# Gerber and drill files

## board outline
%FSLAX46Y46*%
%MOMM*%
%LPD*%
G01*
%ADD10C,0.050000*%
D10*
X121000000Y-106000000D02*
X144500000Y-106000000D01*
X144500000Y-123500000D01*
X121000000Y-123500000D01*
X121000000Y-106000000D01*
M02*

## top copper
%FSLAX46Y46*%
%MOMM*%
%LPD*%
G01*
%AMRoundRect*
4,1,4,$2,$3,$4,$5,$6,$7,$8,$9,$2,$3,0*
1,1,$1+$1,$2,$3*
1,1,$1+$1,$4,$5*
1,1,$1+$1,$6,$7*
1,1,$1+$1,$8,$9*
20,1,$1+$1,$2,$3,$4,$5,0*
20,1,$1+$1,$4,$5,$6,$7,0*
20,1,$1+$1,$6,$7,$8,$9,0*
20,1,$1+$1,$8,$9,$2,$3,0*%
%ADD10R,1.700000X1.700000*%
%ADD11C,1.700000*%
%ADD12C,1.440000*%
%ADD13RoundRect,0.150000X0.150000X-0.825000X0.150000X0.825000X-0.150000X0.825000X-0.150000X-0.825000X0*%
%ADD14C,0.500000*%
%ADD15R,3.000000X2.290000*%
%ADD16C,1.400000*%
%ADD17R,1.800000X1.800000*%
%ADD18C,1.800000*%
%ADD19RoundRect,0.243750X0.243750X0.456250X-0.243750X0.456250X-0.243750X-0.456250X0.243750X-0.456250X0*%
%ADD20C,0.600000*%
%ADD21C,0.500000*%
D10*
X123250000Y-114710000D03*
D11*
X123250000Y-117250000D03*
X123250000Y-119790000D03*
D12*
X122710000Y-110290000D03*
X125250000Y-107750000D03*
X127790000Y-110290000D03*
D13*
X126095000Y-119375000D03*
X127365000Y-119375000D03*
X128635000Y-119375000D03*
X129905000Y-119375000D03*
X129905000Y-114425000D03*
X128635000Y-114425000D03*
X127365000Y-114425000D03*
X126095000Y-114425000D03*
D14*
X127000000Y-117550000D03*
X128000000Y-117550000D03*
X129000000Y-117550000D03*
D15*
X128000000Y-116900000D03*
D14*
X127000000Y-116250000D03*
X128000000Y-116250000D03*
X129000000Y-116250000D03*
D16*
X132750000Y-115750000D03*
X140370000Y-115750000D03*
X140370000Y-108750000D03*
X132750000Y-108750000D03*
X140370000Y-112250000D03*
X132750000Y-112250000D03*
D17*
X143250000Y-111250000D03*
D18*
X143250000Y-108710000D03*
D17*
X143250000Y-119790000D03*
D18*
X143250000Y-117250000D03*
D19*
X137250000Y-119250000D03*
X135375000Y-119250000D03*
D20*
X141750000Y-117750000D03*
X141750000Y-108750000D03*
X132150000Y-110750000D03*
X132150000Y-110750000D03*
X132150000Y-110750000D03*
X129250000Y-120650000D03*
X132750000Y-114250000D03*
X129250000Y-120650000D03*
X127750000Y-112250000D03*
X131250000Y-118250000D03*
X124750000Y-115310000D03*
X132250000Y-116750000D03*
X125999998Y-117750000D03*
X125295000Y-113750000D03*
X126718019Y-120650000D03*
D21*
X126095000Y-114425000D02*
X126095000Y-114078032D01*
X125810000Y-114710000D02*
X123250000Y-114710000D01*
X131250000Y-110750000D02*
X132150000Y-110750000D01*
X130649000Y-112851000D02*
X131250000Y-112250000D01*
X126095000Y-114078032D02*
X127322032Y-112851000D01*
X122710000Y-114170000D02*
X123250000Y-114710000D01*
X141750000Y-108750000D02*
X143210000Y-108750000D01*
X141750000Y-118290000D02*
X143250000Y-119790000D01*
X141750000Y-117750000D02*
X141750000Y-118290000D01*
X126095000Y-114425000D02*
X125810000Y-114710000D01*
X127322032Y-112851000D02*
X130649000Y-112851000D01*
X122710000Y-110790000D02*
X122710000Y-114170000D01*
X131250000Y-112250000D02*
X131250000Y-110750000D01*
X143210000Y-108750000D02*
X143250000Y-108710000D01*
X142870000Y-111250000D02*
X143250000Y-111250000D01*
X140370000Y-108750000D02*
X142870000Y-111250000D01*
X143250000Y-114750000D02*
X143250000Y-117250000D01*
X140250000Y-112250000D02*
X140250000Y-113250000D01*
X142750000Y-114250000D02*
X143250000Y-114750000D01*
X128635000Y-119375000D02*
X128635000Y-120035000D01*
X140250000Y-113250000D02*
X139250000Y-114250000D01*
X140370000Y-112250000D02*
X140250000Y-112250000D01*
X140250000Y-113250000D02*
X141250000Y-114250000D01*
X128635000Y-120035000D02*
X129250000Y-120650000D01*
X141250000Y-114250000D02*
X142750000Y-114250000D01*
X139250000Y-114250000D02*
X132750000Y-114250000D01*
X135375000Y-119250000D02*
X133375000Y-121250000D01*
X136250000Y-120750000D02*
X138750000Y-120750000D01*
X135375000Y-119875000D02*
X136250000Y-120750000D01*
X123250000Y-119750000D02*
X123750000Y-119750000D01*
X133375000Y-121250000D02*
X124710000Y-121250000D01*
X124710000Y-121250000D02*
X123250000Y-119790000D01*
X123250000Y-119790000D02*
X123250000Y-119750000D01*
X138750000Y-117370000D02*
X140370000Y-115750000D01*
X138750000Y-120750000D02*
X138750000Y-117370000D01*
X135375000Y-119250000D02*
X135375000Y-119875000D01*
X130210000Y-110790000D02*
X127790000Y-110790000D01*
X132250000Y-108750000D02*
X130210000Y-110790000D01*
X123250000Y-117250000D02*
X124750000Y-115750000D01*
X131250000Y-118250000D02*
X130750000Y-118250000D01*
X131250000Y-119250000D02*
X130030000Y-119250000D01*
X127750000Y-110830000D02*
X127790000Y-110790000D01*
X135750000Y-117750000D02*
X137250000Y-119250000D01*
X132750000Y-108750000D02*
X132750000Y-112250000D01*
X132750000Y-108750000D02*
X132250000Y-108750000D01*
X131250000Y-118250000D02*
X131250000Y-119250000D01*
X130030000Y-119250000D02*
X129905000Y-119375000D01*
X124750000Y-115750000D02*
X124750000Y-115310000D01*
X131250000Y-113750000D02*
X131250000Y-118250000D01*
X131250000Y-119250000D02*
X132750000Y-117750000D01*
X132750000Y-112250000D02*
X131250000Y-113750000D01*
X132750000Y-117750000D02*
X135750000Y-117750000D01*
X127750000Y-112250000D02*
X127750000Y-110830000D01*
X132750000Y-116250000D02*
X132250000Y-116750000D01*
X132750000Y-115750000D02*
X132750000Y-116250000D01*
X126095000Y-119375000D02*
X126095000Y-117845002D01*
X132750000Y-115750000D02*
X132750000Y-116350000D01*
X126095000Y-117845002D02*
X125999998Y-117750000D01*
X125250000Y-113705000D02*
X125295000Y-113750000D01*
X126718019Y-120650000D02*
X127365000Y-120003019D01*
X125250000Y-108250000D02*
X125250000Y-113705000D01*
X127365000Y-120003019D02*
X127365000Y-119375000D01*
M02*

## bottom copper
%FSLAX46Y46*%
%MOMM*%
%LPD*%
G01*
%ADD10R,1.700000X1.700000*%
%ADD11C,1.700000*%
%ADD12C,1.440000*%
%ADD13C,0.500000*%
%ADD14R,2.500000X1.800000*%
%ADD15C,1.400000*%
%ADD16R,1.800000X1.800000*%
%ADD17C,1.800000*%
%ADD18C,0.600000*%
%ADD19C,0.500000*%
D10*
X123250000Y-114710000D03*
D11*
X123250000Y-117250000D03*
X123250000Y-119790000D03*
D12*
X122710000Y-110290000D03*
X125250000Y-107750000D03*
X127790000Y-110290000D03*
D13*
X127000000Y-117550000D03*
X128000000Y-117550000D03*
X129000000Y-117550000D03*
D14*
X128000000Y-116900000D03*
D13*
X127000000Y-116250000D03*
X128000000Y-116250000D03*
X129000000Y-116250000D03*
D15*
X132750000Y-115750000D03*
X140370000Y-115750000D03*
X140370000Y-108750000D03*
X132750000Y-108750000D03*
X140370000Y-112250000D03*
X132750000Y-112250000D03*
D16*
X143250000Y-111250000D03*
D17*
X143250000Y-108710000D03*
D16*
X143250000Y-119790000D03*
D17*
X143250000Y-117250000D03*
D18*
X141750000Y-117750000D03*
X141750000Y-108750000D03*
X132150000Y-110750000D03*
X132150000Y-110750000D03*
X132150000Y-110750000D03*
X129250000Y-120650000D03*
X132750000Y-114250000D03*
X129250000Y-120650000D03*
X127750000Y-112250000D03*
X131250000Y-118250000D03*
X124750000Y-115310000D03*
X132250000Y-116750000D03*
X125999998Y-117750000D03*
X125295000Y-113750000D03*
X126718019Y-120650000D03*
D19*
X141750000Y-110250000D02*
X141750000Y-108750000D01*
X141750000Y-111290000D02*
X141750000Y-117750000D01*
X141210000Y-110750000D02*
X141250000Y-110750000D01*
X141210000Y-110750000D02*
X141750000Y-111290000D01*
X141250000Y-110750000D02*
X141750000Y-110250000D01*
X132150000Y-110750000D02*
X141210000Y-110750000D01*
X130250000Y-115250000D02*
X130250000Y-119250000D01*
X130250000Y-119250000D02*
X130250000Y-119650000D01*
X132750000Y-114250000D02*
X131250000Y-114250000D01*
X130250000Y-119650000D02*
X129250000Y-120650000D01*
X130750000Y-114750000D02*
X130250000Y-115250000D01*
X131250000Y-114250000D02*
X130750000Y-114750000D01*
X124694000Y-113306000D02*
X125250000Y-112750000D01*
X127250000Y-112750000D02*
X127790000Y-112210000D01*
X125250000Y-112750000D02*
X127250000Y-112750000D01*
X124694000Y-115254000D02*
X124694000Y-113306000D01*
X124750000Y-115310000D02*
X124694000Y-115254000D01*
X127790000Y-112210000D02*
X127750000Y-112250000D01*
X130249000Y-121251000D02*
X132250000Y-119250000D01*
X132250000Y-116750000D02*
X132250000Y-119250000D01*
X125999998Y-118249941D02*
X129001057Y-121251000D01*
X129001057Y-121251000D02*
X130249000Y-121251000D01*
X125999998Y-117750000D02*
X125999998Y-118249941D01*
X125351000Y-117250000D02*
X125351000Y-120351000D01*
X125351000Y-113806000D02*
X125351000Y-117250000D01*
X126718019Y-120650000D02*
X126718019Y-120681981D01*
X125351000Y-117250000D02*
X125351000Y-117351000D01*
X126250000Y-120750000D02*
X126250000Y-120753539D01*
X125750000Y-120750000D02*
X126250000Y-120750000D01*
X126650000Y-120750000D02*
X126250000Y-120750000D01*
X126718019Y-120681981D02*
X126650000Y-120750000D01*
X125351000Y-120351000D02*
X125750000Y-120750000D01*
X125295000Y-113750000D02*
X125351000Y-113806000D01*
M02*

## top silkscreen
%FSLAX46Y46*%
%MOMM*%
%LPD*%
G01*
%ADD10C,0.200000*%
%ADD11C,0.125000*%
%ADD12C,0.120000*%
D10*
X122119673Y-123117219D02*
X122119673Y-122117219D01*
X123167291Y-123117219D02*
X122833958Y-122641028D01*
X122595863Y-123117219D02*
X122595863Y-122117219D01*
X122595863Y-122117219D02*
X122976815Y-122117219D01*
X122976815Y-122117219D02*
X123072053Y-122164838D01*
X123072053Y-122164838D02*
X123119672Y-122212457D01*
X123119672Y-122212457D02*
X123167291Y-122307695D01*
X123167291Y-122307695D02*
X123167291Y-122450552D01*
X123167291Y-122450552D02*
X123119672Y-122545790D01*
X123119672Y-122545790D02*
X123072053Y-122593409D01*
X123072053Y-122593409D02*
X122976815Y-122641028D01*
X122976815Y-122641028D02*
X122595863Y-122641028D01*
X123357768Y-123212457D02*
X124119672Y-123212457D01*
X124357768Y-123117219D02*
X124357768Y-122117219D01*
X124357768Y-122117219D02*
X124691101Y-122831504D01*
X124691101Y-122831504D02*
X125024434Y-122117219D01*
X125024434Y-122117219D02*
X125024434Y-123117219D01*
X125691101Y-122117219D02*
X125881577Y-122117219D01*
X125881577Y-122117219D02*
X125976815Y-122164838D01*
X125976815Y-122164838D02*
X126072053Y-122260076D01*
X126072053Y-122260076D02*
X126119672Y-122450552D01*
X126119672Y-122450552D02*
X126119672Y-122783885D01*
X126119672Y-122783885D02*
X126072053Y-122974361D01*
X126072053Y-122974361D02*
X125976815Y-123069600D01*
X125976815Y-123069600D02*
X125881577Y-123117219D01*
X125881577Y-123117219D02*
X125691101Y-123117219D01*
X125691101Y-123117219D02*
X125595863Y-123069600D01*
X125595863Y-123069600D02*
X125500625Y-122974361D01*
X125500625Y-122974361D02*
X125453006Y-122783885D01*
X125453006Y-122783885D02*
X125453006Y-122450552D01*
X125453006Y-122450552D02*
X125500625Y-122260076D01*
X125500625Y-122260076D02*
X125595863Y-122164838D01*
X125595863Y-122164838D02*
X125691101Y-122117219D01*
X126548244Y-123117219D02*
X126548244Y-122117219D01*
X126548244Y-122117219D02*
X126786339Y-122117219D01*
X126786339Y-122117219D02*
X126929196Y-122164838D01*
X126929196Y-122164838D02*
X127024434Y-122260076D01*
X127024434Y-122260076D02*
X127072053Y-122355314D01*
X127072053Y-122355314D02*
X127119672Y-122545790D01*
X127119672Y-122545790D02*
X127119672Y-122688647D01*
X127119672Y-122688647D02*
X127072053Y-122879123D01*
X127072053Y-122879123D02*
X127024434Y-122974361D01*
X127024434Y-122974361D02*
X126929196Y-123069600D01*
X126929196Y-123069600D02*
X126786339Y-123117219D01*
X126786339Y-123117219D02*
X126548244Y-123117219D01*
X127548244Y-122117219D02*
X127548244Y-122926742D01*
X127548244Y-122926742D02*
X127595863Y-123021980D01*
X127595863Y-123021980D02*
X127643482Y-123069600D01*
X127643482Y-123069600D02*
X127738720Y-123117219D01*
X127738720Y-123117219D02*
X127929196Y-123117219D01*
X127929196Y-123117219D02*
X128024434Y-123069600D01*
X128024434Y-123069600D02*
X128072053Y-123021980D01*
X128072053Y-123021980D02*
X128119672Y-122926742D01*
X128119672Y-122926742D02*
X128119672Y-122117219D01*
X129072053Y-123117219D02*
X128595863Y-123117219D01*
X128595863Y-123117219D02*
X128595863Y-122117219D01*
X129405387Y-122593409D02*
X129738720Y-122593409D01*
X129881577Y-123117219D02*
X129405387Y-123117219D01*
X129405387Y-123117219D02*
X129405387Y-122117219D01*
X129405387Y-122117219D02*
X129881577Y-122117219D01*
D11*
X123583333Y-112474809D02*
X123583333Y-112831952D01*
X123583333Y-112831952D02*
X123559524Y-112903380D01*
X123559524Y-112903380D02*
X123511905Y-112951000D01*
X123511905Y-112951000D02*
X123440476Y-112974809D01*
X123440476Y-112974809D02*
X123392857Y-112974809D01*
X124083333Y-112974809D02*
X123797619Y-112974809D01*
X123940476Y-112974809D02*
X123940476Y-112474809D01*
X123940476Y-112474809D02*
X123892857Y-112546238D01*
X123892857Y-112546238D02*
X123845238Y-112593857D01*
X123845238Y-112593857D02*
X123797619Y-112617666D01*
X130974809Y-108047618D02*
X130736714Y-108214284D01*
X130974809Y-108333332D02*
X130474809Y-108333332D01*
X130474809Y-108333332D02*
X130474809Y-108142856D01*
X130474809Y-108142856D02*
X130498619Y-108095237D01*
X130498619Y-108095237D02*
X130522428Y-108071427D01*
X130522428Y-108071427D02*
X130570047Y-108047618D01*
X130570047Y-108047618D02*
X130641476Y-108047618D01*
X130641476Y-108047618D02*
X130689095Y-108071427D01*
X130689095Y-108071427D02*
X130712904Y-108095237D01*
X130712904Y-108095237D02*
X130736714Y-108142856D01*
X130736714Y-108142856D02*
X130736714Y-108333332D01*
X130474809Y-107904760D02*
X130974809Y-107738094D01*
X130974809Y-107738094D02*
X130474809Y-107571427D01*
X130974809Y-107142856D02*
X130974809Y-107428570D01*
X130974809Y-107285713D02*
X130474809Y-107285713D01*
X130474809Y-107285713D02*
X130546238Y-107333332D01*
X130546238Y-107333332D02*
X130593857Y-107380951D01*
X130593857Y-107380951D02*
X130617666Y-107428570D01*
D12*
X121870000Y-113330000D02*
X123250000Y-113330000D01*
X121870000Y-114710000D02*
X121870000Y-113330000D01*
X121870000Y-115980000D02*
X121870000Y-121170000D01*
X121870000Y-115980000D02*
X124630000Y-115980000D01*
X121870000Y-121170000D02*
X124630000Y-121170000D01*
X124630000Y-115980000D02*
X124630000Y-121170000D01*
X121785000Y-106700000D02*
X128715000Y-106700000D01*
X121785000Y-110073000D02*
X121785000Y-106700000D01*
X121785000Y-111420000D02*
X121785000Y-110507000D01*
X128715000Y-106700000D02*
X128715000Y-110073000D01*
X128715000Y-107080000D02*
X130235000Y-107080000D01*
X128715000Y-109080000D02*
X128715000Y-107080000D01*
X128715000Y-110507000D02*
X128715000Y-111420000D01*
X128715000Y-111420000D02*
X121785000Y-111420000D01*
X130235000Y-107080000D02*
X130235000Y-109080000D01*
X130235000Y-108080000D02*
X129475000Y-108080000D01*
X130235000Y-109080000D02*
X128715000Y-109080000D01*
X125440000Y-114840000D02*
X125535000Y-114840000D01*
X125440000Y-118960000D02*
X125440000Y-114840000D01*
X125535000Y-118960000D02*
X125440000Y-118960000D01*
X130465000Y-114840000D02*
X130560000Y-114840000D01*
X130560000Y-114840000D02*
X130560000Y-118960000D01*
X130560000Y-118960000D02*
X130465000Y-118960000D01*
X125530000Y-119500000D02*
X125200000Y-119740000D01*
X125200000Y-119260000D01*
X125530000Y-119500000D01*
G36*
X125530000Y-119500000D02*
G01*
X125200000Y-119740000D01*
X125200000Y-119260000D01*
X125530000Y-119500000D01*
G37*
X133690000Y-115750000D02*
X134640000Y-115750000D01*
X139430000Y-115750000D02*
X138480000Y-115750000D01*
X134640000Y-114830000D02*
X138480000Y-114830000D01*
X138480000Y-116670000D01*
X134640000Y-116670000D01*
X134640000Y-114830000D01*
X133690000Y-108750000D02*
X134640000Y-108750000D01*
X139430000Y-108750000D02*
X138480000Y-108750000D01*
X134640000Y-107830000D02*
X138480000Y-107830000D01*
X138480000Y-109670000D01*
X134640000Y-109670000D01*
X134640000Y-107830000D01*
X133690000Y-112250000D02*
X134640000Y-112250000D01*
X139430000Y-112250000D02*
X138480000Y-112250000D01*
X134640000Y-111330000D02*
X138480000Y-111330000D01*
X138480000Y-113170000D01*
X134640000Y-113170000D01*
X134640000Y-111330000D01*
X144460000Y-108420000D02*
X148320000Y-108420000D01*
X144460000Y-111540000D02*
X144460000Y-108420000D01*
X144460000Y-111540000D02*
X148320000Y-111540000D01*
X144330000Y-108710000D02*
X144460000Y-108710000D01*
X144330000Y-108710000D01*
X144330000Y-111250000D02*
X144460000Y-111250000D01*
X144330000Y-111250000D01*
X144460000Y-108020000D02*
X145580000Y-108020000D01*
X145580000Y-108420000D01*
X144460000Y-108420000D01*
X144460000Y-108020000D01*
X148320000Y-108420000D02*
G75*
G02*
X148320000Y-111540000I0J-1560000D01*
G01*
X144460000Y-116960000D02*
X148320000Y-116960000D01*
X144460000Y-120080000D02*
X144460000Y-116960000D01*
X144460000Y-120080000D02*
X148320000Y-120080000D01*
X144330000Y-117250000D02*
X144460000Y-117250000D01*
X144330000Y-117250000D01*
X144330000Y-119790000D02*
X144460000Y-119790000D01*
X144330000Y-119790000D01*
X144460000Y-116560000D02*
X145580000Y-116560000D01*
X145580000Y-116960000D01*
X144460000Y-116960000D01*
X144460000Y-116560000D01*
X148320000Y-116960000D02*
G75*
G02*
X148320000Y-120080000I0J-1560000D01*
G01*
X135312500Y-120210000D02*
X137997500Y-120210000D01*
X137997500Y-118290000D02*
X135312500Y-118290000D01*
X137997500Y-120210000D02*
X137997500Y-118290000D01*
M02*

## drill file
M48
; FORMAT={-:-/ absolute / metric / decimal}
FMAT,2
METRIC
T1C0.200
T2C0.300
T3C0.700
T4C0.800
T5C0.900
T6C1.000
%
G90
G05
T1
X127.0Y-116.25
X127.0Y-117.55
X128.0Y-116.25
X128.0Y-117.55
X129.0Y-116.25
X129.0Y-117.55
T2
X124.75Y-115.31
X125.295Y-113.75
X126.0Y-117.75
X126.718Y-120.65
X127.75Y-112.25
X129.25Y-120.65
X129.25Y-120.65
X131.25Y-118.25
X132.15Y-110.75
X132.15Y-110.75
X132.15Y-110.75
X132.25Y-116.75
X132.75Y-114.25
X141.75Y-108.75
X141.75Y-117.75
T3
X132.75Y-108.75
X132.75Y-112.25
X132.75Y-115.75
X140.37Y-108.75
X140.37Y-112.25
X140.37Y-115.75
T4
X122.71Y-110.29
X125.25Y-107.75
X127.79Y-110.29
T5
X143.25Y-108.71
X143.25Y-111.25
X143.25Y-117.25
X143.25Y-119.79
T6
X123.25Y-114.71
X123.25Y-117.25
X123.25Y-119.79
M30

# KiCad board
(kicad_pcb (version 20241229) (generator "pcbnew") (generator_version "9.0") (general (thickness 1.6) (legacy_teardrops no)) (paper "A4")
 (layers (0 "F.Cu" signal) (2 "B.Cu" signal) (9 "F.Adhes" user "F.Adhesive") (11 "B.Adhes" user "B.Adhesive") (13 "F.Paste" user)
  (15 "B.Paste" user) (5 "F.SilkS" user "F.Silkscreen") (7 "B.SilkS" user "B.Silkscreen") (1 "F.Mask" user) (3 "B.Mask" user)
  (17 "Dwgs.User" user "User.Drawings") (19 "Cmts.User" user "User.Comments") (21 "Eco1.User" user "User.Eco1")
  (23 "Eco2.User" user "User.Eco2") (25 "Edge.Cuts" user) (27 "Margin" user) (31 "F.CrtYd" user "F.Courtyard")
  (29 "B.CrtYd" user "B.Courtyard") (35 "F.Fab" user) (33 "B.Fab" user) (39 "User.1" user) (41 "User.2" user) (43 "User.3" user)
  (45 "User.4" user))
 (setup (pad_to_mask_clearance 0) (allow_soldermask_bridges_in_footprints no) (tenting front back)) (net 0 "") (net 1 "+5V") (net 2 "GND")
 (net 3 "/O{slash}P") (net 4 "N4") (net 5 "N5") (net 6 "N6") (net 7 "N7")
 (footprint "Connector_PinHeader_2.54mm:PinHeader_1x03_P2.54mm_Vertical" (layer "F.Cu") (at 123.25 114.71)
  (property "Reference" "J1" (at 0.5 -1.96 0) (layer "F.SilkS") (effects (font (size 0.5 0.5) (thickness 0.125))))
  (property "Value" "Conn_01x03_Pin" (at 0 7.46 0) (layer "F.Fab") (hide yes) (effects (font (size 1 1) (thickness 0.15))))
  (fp_line (start -1.38 -1.38) (end 0 -1.38) (stroke (width 0.12) (type solid)) (layer "F.SilkS"))
  (fp_line (start -1.38 0) (end -1.38 -1.38) (stroke (width 0.12) (type solid)) (layer "F.SilkS"))
  (fp_line (start -1.38 1.27) (end -1.38 6.46) (stroke (width 0.12) (type solid)) (layer "F.SilkS"))
  (fp_line (start -1.38 1.27) (end 1.38 1.27) (stroke (width 0.12) (type solid)) (layer "F.SilkS"))
  (fp_line (start -1.38 6.46) (end 1.38 6.46) (stroke (width 0.12) (type solid)) (layer "F.SilkS"))
  (fp_line (start 1.38 1.27) (end 1.38 6.46) (stroke (width 0.12) (type solid)) (layer "F.SilkS"))
  (pad "1" thru_hole rect (at 0 0) (size 1.7 1.7) (drill 1) (layers "*.Cu" "*.Mask") (remove_unused_layers no) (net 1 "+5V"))
  (pad "2" thru_hole circle (at 0 2.54) (size 1.7 1.7) (drill 1) (layers "*.Cu" "*.Mask") (remove_unused_layers no) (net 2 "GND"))
  (pad "3" thru_hole circle (at 0 5.08) (size 1.7 1.7) (drill 1) (layers "*.Cu" "*.Mask") (remove_unused_layers no) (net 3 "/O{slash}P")))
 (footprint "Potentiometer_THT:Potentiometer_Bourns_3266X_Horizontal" (layer "F.Cu") (at 122.71 110.29 180)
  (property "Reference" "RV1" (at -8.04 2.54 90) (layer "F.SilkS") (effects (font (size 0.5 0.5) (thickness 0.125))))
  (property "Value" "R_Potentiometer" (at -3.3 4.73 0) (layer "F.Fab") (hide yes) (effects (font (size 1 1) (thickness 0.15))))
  (fp_line (start 0.925 3.59) (end -6.005 3.59) (stroke (width 0.12) (type solid)) (layer "F.SilkS"))
  (fp_line (start 0.925 0.217) (end 0.925 3.59) (stroke (width 0.12) (type solid)) (layer "F.SilkS"))
  (fp_line (start 0.925 -1.13) (end 0.925 -0.217) (stroke (width 0.12) (type solid)) (layer "F.SilkS"))
  (fp_line (start -6.005 3.59) (end -6.005 0.217) (stroke (width 0.12) (type solid)) (layer "F.SilkS"))
  (fp_line (start -6.005 3.21) (end -7.525 3.21) (stroke (width 0.12) (type solid)) (layer "F.SilkS"))
  (fp_line (start -6.005 1.21) (end -6.005 3.21) (stroke (width 0.12) (type solid)) (layer "F.SilkS"))
  (fp_line (start -6.005 -0.217) (end -6.005 -1.13) (stroke (width 0.12) (type solid)) (layer "F.SilkS"))
  (fp_line (start -6.005 -1.13) (end 0.925 -1.13) (stroke (width 0.12) (type solid)) (layer "F.SilkS"))
  (fp_line (start -7.525 3.21) (end -7.525 1.21) (stroke (width 0.12) (type solid)) (layer "F.SilkS"))
  (fp_line (start -7.525 2.21) (end -6.765 2.21) (stroke (width 0.12) (type solid)) (layer "F.SilkS"))
  (fp_line (start -7.525 1.21) (end -6.005 1.21) (stroke (width 0.12) (type solid)) (layer "F.SilkS"))
  (pad "1" thru_hole circle (at 0 0 180) (size 1.44 1.44) (drill 0.8) (layers "*.Cu" "*.Mask") (remove_unused_layers no) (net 1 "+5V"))
  (pad "2" thru_hole circle (at -2.54 2.54 180) (size 1.44 1.44) (drill 0.8) (layers "*.Cu" "*.Mask") (remove_unused_layers no) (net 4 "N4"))
  (pad "3" thru_hole circle (at -5.08 0 180) (size 1.44 1.44) (drill 0.8) (layers "*.Cu" "*.Mask") (remove_unused_layers no) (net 2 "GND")))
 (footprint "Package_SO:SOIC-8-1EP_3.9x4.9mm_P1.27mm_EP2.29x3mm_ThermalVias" (layer "F.Cu") (at 128 116.9 90)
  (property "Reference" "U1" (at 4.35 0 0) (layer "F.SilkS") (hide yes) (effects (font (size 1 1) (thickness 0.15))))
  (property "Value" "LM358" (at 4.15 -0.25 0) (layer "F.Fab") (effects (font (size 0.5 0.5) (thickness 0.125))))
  (fp_line (start 2.06 -2.56) (end 2.06 -2.465) (stroke (width 0.12) (type solid)) (layer "F.SilkS"))
  (fp_line (start -2.06 -2.56) (end 2.06 -2.56) (stroke (width 0.12) (type solid)) (layer "F.SilkS"))
  (fp_line (start -2.06 -2.465) (end -2.06 -2.56) (stroke (width 0.12) (type solid)) (layer "F.SilkS"))
  (fp_line (start 2.06 2.465) (end 2.06 2.56) (stroke (width 0.12) (type solid)) (layer "F.SilkS"))
  (fp_line (start 2.06 2.56) (end -2.06 2.56) (stroke (width 0.12) (type solid)) (layer "F.SilkS"))
  (fp_line (start -2.06 2.56) (end -2.06 2.465) (stroke (width 0.12) (type solid)) (layer "F.SilkS"))
  (fp_poly (pts (xy -2.6 -2.47) (xy -2.84 -2.8) (xy -2.36 -2.8)) (stroke (width 0.12) (type solid)) (fill yes) (layer "F.SilkS"))
  (pad "" smd roundrect (at -0.57 -0.75 90) (size 0.96 1.25) (layers "F.Paste") (roundrect_rratio 0.25))
  (pad "" smd roundrect (at -0.57 0.75 90) (size 0.96 1.25) (layers "F.Paste") (roundrect_rratio 0.25))
  (pad "" smd roundrect (at 0.57 -0.75 90) (size 0.96 1.25) (layers "F.Paste") (roundrect_rratio 0.25))
  (pad "" smd roundrect (at 0.57 0.75 90) (size 0.96 1.25) (layers "F.Paste") (roundrect_rratio 0.25))
  (pad "1" smd roundrect (at -2.475 -1.905 90) (size 1.95 0.6) (layers "F.Cu" "F.Mask" "F.Paste") (roundrect_rratio 0.25) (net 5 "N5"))
  (pad "2" smd roundrect (at -2.475 -0.635 90) (size 1.95 0.6) (layers "F.Cu" "F.Mask" "F.Paste") (roundrect_rratio 0.25) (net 4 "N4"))
  (pad "3" smd roundrect (at -2.475 0.635 90) (size 1.95 0.6) (layers "F.Cu" "F.Mask" "F.Paste") (roundrect_rratio 0.25) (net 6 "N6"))
  (pad "4" smd roundrect (at -2.475 1.905 90) (size 1.95 0.6) (layers "F.Cu" "F.Mask" "F.Paste") (roundrect_rratio 0.25) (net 2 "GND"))
  (pad "5" smd roundrect (at 2.475 1.905 90) (size 1.95 0.6) (layers "F.Cu" "F.Mask" "F.Paste") (roundrect_rratio 0.25))
  (pad "6" smd roundrect (at 2.475 0.635 90) (size 1.95 0.6) (layers "F.Cu" "F.Mask" "F.Paste") (roundrect_rratio 0.25))
  (pad "7" smd roundrect (at 2.475 -0.635 90) (size 1.95 0.6) (layers "F.Cu" "F.Mask" "F.Paste") (roundrect_rratio 0.25))
  (pad "8" smd roundrect (at 2.475 -1.905 90) (size 1.95 0.6) (layers "F.Cu" "F.Mask" "F.Paste") (roundrect_rratio 0.25) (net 1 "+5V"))
  (pad "9" thru_hole circle (at -0.65 -1 90) (size 0.5 0.5) (drill 0.2) (layers "*.Cu") (remove_unused_layers no))
  (pad "9" thru_hole circle (at -0.65 0 90) (size 0.5 0.5) (drill 0.2) (layers "*.Cu") (remove_unused_layers no))
  (pad "9" thru_hole circle (at -0.65 1 90) (size 0.5 0.5) (drill 0.2) (layers "*.Cu") (remove_unused_layers no))
  (pad "9" smd rect (at 0 0 90) (size 1.8 2.5) (layers "B.Cu") (zone_connect 2))
  (pad "9" smd rect (at 0 0 90) (size 2.29 3) (layers "F.Cu" "F.Mask") (zone_connect 2))
  (pad "9" thru_hole circle (at 0.65 -1 90) (size 0.5 0.5) (drill 0.2) (layers "*.Cu") (remove_unused_layers no))
  (pad "9" thru_hole circle (at 0.65 0 90) (size 0.5 0.5) (drill 0.2) (layers "*.Cu") (remove_unused_layers no))
  (pad "9" thru_hole circle (at 0.65 1 90) (size 0.5 0.5) (drill 0.2) (layers "*.Cu") (remove_unused_layers no)))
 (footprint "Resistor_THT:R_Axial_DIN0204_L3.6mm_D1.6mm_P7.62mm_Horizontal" (layer "F.Cu") (at 132.75 115.75)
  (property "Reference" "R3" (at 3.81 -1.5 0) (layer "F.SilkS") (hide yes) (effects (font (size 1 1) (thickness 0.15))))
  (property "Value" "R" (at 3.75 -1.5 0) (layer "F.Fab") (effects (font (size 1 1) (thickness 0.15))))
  (fp_line (start 0.94 0) (end 1.89 0) (stroke (width 0.12) (type solid)) (layer "F.SilkS"))
  (fp_line (start 6.68 0) (end 5.73 0) (stroke (width 0.12) (type solid)) (layer "F.SilkS"))
  (fp_rect (start 1.89 -0.92) (end 5.73 0.92) (stroke (width 0.12) (type solid)) (fill no) (layer "F.SilkS"))
  (pad "1" thru_hole circle (at 0 0) (size 1.4 1.4) (drill 0.7) (layers "*.Cu" "*.Mask") (remove_unused_layers no) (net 5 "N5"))
  (pad "2" thru_hole circle (at 7.62 0) (size 1.4 1.4) (drill 0.7) (layers "*.Cu" "*.Mask") (remove_unused_layers no) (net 3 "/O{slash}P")))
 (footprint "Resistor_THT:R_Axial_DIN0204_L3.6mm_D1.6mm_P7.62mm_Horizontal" (layer "F.Cu") (at 140.37 108.75 180)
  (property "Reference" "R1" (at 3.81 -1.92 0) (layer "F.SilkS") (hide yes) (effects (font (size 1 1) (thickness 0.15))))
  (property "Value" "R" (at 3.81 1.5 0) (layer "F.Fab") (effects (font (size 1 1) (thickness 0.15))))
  (fp_line (start 6.68 0) (end 5.73 0) (stroke (width 0.12) (type solid)) (layer "F.SilkS"))
  (fp_line (start 0.94 0) (end 1.89 0) (stroke (width 0.12) (type solid)) (layer "F.SilkS"))
  (fp_rect (start 1.89 -0.92) (end 5.73 0.92) (stroke (width 0.12) (type solid)) (fill no) (layer "F.SilkS"))
  (pad "1" thru_hole circle (at 0 0 180) (size 1.4 1.4) (drill 0.7) (layers "*.Cu" "*.Mask") (remove_unused_layers no) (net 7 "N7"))
  (pad "2" thru_hole circle (at 7.62 0 180) (size 1.4 1.4) (drill 0.7) (layers "*.Cu" "*.Mask") (remove_unused_layers no) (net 2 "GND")))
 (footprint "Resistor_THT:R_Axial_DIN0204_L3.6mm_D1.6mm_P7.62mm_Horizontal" (layer "F.Cu") (at 140.37 112.25 180)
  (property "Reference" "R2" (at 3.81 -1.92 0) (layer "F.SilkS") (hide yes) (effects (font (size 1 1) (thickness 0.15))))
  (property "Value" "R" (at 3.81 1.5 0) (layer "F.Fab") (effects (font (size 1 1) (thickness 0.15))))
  (fp_line (start 6.68 0) (end 5.73 0) (stroke (width 0.12) (type solid)) (layer "F.SilkS"))
  (fp_line (start 0.94 0) (end 1.89 0) (stroke (width 0.12) (type solid)) (layer "F.SilkS"))
  (fp_rect (start 1.89 -0.92) (end 5.73 0.92) (stroke (width 0.12) (type solid)) (fill no) (layer "F.SilkS"))
  (pad "1" thru_hole circle (at 0 0 180) (size 1.4 1.4) (drill 0.7) (layers "*.Cu" "*.Mask") (remove_unused_layers no) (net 6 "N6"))
  (pad "2" thru_hole circle (at 7.62 0 180) (size 1.4 1.4) (drill 0.7) (layers "*.Cu" "*.Mask") (remove_unused_layers no) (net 2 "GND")))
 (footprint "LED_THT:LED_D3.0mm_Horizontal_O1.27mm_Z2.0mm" (layer "F.Cu") (at 143.25 111.25 90)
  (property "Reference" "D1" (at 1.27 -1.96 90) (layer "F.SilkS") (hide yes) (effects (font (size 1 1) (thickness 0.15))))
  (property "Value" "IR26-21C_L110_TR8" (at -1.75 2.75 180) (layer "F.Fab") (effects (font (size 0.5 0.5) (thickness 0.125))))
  (fp_line (start 2.83 1.21) (end 2.83 5.07) (stroke (width 0.12) (type solid)) (layer "F.SilkS"))
  (fp_line (start -0.29 1.21) (end 2.83 1.21) (stroke (width 0.12) (type solid)) (layer "F.SilkS"))
  (fp_line (start -0.29 1.21) (end -0.29 5.07) (stroke (width 0.12) (type solid)) (layer "F.SilkS"))
  (fp_rect (start 2.54 1.08) (end 2.54 1.21) (stroke (width 0.12) (type solid)) (fill no) (layer "F.SilkS"))
  (fp_rect (start 0 1.08) (end 0 1.21) (stroke (width 0.12) (type solid)) (fill no) (layer "F.SilkS"))
  (fp_rect (start 2.83 1.21) (end 3.23 2.33) (stroke (width 0.12) (type solid)) (fill no) (layer "F.SilkS"))
  (fp_arc (start 2.83 5.07) (mid 1.27 6.63) (end -0.29 5.07) (stroke (width 0.12) (type solid)) (layer "F.SilkS"))
  (pad "1" thru_hole rect (at 0 0 90) (size 1.8 1.8) (drill 0.9) (layers "*.Cu" "*.Mask") (remove_unused_layers no) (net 7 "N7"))
  (pad "2" thru_hole circle (at 2.54 0 90) (size 1.8 1.8) (drill 0.9) (layers "*.Cu" "*.Mask") (remove_unused_layers no) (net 1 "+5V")))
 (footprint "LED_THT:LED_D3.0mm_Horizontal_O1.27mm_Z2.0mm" (layer "F.Cu") (at 143.25 119.79 90)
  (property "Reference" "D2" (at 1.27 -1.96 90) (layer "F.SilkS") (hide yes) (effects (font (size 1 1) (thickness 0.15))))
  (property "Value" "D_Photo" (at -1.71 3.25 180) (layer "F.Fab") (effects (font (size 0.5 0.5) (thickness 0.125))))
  (fp_line (start 2.83 1.21) (end 2.83 5.07) (stroke (width 0.12) (type solid)) (layer "F.SilkS"))
  (fp_line (start -0.29 1.21) (end 2.83 1.21) (stroke (width 0.12) (type solid)) (layer "F.SilkS"))
  (fp_line (start -0.29 1.21) (end -0.29 5.07) (stroke (width 0.12) (type solid)) (layer "F.SilkS"))
  (fp_rect (start 2.54 1.08) (end 2.54 1.21) (stroke (width 0.12) (type solid)) (fill no) (layer "F.SilkS"))
  (fp_rect (start 0 1.08) (end 0 1.21) (stroke (width 0.12) (type solid)) (fill no) (layer "F.SilkS"))
  (fp_rect (start 2.83 1.21) (end 3.23 2.33) (stroke (width 0.12) (type solid)) (fill no) (layer "F.SilkS"))
  (fp_arc (start 2.83 5.07) (mid 1.27 6.63) (end -0.29 5.07) (stroke (width 0.12) (type solid)) (layer "F.SilkS"))
  (pad "1" thru_hole rect (at 0 0 90) (size 1.8 1.8) (drill 0.9) (layers "*.Cu" "*.Mask") (remove_unused_layers no) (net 1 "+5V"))
  (pad "2" thru_hole circle (at 2.54 0 90) (size 1.8 1.8) (drill 0.9) (layers "*.Cu" "*.Mask") (remove_unused_layers no) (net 6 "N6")))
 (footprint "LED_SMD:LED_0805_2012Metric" (layer "F.Cu") (at 136.3125 119.25 180)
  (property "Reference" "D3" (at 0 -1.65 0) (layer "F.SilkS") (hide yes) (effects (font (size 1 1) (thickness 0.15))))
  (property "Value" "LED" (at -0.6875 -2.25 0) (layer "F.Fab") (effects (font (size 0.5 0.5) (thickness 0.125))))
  (fp_line (start 1 -0.96) (end -1.685 -0.96) (stroke (width 0.12) (type solid)) (layer "F.SilkS"))
  (fp_line (start -1.685 0.96) (end 1 0.96) (stroke (width 0.12) (type solid)) (layer "F.SilkS"))
  (fp_line (start -1.685 -0.96) (end -1.685 0.96) (stroke (width 0.12) (type solid)) (layer "F.SilkS"))
  (pad "1" smd roundrect (at -0.9375 0 180) (size 0.975 1.4) (layers "F.Cu" "F.Mask" "F.Paste") (roundrect_rratio 0.25) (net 2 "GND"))
  (pad "2" smd roundrect (at 0.9375 0 180) (size 0.975 1.4) (layers "F.Cu" "F.Mask" "F.Paste") (roundrect_rratio 0.25) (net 3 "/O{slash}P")))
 (gr_rect (start 121 106) (end 144.5 123.5) (stroke (width 0.05) (type default)) (fill no) (layer "Edge.Cuts"))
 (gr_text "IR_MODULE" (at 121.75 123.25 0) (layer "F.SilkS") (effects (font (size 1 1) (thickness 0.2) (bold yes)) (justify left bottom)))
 (segment (start 126.095 114.425) (end 126.095 114.078032) (width 0.5) (layer "F.Cu") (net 1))
 (segment (start 125.81 114.71) (end 123.25 114.71) (width 0.5) (layer "F.Cu") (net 1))
 (segment (start 131.25 110.75) (end 132.15 110.75) (width 0.5) (layer "F.Cu") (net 1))
 (segment (start 130.649 112.851) (end 131.25 112.25) (width 0.5) (layer "F.Cu") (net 1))
 (segment (start 126.095 114.078032) (end 127.322032 112.851) (width 0.5) (layer "F.Cu") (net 1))
 (segment (start 122.71 114.17) (end 123.25 114.71) (width 0.5) (layer "F.Cu") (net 1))
 (segment (start 141.75 108.75) (end 143.21 108.75) (width 0.5) (layer "F.Cu") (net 1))
 (segment (start 141.75 118.29) (end 143.25 119.79) (width 0.5) (layer "F.Cu") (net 1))
 (segment (start 141.75 117.75) (end 141.75 118.29) (width 0.5) (layer "F.Cu") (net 1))
 (segment (start 126.095 114.425) (end 125.81 114.71) (width 0.5) (layer "F.Cu") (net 1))
 (segment (start 127.322032 112.851) (end 130.649 112.851) (width 0.5) (layer "F.Cu") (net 1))
 (segment (start 122.71 110.79) (end 122.71 114.17) (width 0.5) (layer "F.Cu") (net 1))
 (segment (start 131.25 112.25) (end 131.25 110.75) (width 0.5) (layer "F.Cu") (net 1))
 (segment (start 143.21 108.75) (end 143.25 108.71) (width 0.5) (layer "F.Cu") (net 1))
 (via (at 141.75 117.75) (size 0.6) (drill 0.3) (layers "F.Cu" "B.Cu") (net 1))
 (via (at 141.75 108.75) (size 0.6) (drill 0.3) (layers "F.Cu" "B.Cu") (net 1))
 (via (at 132.15 110.75) (size 0.6) (drill 0.3) (layers "F.Cu" "B.Cu") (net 1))
 (via (at 132.15 110.75) (size 0.6) (drill 0.3) (layers "F.Cu" "B.Cu") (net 1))
 (via (at 132.15 110.75) (size 0.6) (drill 0.3) (layers "F.Cu" "B.Cu") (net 1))
 (segment (start 141.75 110.25) (end 141.75 108.75) (width 0.5) (layer "B.Cu") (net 1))
 (segment (start 141.75 111.29) (end 141.75 117.75) (width 0.5) (layer "B.Cu") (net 1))
 (segment (start 141.21 110.75) (end 141.25 110.75) (width 0.5) (layer "B.Cu") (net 1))
 (segment (start 141.21 110.75) (end 141.75 111.29) (width 0.5) (layer "B.Cu") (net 1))
 (segment (start 141.25 110.75) (end 141.75 110.25) (width 0.5) (layer "B.Cu") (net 1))
 (segment (start 132.15 110.75) (end 141.21 110.75) (width 0.5) (layer "B.Cu") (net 1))
 (segment (start 142.87 111.25) (end 143.25 111.25) (width 0.5) (layer "F.Cu") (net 7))
 (segment (start 140.37 108.75) (end 142.87 111.25) (width 0.5) (layer "F.Cu") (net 7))
 (segment (start 143.25 114.75) (end 143.25 117.25) (width 0.5) (layer "F.Cu") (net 6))
 (segment (start 140.25 112.25) (end 140.25 113.25) (width 0.5) (layer "F.Cu") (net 6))
 (segment (start 142.75 114.25) (end 143.25 114.75) (width 0.5) (layer "F.Cu") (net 6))
 (segment (start 128.635 119.375) (end 128.635 120.035) (width 0.5) (layer "F.Cu") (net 6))
 (segment (start 140.25 113.25) (end 139.25 114.25) (width 0.5) (layer "F.Cu") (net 6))
 (segment (start 140.37 112.25) (end 140.25 112.25) (width 0.5) (layer "F.Cu") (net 6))
 (segment (start 140.25 113.25) (end 141.25 114.25) (width 0.5) (layer "F.Cu") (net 6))
 (segment (start 128.635 120.035) (end 129.25 120.65) (width 0.5) (layer "F.Cu") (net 6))
 (segment (start 141.25 114.25) (end 142.75 114.25) (width 0.5) (layer "F.Cu") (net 6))
 (segment (start 139.25 114.25) (end 132.75 114.25) (width 0.5) (layer "F.Cu") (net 6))
 (via (at 129.25 120.65) (size 0.6) (drill 0.3) (layers "F.Cu" "B.Cu") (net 6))
 (via (at 132.75 114.25) (size 0.6) (drill 0.3) (layers "F.Cu" "B.Cu") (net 6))
 (via (at 129.25 120.65) (size 0.6) (drill 0.3) (layers "F.Cu" "B.Cu") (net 6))
 (segment (start 130.25 115.25) (end 130.25 119.25) (width 0.5) (layer "B.Cu") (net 6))
 (segment (start 130.25 119.25) (end 130.25 119.65) (width 0.5) (layer "B.Cu") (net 6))
 (segment (start 132.75 114.25) (end 131.25 114.25) (width 0.5) (layer "B.Cu") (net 6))
 (segment (start 130.25 119.65) (end 129.25 120.65) (width 0.5) (layer "B.Cu") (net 6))
 (segment (start 130.75 114.75) (end 130.25 115.25) (width 0.5) (layer "B.Cu") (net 6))
 (segment (start 131.25 114.25) (end 130.75 114.75) (width 0.5) (layer "B.Cu") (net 6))
 (segment (start 135.375 119.25) (end 133.375 121.25) (width 0.5) (layer "F.Cu") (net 3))
 (segment (start 136.25 120.75) (end 138.75 120.75) (width 0.5) (layer "F.Cu") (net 3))
 (segment (start 135.375 119.875) (end 136.25 120.75) (width 0.5) (layer "F.Cu") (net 3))
 (segment (start 123.25 119.75) (end 123.75 119.75) (width 0.5) (layer "F.Cu") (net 3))
 (segment (start 133.375 121.25) (end 124.71 121.25) (width 0.5) (layer "F.Cu") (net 3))
 (segment (start 124.71 121.25) (end 123.25 119.79) (width 0.5) (layer "F.Cu") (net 3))
 (segment (start 123.25 119.79) (end 123.25 119.75) (width 0.5) (layer "F.Cu") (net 3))
 (segment (start 138.75 117.37) (end 140.37 115.75) (width 0.5) (layer "F.Cu") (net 3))
 (segment (start 138.75 120.75) (end 138.75 117.37) (width 0.5) (layer "F.Cu") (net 3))
 (segment (start 135.375 119.25) (end 135.375 119.875) (width 0.5) (layer "F.Cu") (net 3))
 (segment (start 130.21 110.79) (end 127.79 110.79) (width 0.5) (layer "F.Cu") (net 2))
 (segment (start 132.25 108.75) (end 130.21 110.79) (width 0.5) (layer "F.Cu") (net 2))
 (segment (start 123.25 117.25) (end 124.75 115.75) (width 0.5) (layer "F.Cu") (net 2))
 (segment (start 131.25 118.25) (end 130.75 118.25) (width 0.5) (layer "F.Cu") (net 2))
 (segment (start 131.25 119.25) (end 130.03 119.25) (width 0.5) (layer "F.Cu") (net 2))
 (segment (start 127.75 110.83) (end 127.79 110.79) (width 0.5) (layer "F.Cu") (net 2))
 (segment (start 135.75 117.75) (end 137.25 119.25) (width 0.5) (layer "F.Cu") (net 2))
 (segment (start 132.75 108.75) (end 132.75 112.25) (width 0.5) (layer "F.Cu") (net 2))
 (segment (start 132.75 108.75) (end 132.25 108.75) (width 0.5) (layer "F.Cu") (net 2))
 (segment (start 131.25 118.25) (end 131.25 119.25) (width 0.5) (layer "F.Cu") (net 2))
 (segment (start 130.03 119.25) (end 129.905 119.375) (width 0.5) (layer "F.Cu") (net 2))
 (segment (start 124.75 115.75) (end 124.75 115.31) (width 0.5) (layer "F.Cu") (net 2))
 (segment (start 131.25 113.75) (end 131.25 118.25) (width 0.5) (layer "F.Cu") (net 2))
 (segment (start 131.25 119.25) (end 132.75 117.75) (width 0.5) (layer "F.Cu") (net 2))
 (segment (start 132.75 112.25) (end 131.25 113.75) (width 0.5) (layer "F.Cu") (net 2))
 (segment (start 132.75 117.75) (end 135.75 117.75) (width 0.5) (layer "F.Cu") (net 2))
 (segment (start 127.75 112.25) (end 127.75 110.83) (width 0.5) (layer "F.Cu") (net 2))
 (via (at 127.75 112.25) (size 0.6) (drill 0.3) (layers "F.Cu" "B.Cu") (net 2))
 (via (at 131.25 118.25) (size 0.6) (drill 0.3) (layers "F.Cu" "B.Cu") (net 2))
 (via (at 124.75 115.31) (size 0.6) (drill 0.3) (layers "F.Cu" "B.Cu") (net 2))
 (segment (start 124.694 113.306) (end 125.25 112.75) (width 0.5) (layer "B.Cu") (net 2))
 (segment (start 127.25 112.75) (end 127.79 112.21) (width 0.5) (layer "B.Cu") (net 2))
 (segment (start 125.25 112.75) (end 127.25 112.75) (width 0.5) (layer "B.Cu") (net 2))
 (segment (start 124.694 115.254) (end 124.694 113.306) (width 0.5) (layer "B.Cu") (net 2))
 (segment (start 124.75 115.31) (end 124.694 115.254) (width 0.5) (layer "B.Cu") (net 2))
 (segment (start 127.79 112.21) (end 127.75 112.25) (width 0.5) (layer "B.Cu") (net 2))
 (segment (start 132.75 116.25) (end 132.25 116.75) (width 0.5) (layer "F.Cu") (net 5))
 (segment (start 132.75 115.75) (end 132.75 116.25) (width 0.5) (layer "F.Cu") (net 5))
 (segment (start 126.095 119.375) (end 126.095 117.845002) (width 0.5) (layer "F.Cu") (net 5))
 (segment (start 132.75 115.75) (end 132.75 116.35) (width 0.5) (layer "F.Cu") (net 5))
 (segment (start 126.095 117.845002) (end 125.999998 117.75) (width 0.5) (layer "F.Cu") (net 5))
 (via (at 132.25 116.75) (size 0.6) (drill 0.3) (layers "F.Cu" "B.Cu") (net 5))
 (via (at 125.999998 117.75) (size 0.6) (drill 0.3) (layers "F.Cu" "B.Cu") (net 5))
 (segment (start 130.249 121.251) (end 132.25 119.25) (width 0.5) (layer "B.Cu") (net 5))
 (segment (start 132.25 116.75) (end 132.25 119.25) (width 0.5) (layer "B.Cu") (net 5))
 (segment (start 125.999998 118.249941) (end 129.001057 121.251) (width 0.5) (layer "B.Cu") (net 5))
 (segment (start 129.001057 121.251) (end 130.249 121.251) (width 0.5) (layer "B.Cu") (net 5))
 (segment (start 125.999998 117.75) (end 125.999998 118.249941) (width 0.5) (layer "B.Cu") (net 5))
 (segment (start 125.25 113.705) (end 125.295 113.75) (width 0.5) (layer "F.Cu") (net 4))
 (segment (start 126.718019 120.65) (end 127.365 120.003019) (width 0.5) (layer "F.Cu") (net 4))
 (segment (start 125.25 108.25) (end 125.25 113.705) (width 0.5) (layer "F.Cu") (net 4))
 (segment (start 127.365 120.003019) (end 127.365 119.375) (width 0.5) (layer "F.Cu") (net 4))
 (via (at 125.295 113.75) (size 0.6) (drill 0.3) (layers "F.Cu" "B.Cu") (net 4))
 (via (at 126.718019 120.65) (size 0.6) (drill 0.3) (layers "F.Cu" "B.Cu") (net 4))
 (segment (start 125.351 117.25) (end 125.351 120.351) (width 0.5) (layer "B.Cu") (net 4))
 (segment (start 125.351 113.806) (end 125.351 117.25) (width 0.5) (layer "B.Cu") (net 4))
 (segment (start 126.718019 120.65) (end 126.718019 120.681981) (width 0.5) (layer "B.Cu") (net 4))
 (segment (start 125.351 117.25) (end 125.351 117.351) (width 0.5) (layer "B.Cu") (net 4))
 (segment (start 126.25 120.75) (end 126.25 120.753539) (width 0.5) (layer "B.Cu") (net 4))
 (segment (start 125.75 120.75) (end 126.25 120.75) (width 0.5) (layer "B.Cu") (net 4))
 (segment (start 126.65 120.75) (end 126.25 120.75) (width 0.5) (layer "B.Cu") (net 4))
 (segment (start 126.718019 120.681981) (end 126.65 120.75) (width 0.5) (layer "B.Cu") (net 4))
 (segment (start 125.351 120.351) (end 125.75 120.75) (width 0.5) (layer "B.Cu") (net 4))
 (segment (start 125.295 113.75) (end 125.351 113.806) (width 0.5) (layer "B.Cu") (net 4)))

